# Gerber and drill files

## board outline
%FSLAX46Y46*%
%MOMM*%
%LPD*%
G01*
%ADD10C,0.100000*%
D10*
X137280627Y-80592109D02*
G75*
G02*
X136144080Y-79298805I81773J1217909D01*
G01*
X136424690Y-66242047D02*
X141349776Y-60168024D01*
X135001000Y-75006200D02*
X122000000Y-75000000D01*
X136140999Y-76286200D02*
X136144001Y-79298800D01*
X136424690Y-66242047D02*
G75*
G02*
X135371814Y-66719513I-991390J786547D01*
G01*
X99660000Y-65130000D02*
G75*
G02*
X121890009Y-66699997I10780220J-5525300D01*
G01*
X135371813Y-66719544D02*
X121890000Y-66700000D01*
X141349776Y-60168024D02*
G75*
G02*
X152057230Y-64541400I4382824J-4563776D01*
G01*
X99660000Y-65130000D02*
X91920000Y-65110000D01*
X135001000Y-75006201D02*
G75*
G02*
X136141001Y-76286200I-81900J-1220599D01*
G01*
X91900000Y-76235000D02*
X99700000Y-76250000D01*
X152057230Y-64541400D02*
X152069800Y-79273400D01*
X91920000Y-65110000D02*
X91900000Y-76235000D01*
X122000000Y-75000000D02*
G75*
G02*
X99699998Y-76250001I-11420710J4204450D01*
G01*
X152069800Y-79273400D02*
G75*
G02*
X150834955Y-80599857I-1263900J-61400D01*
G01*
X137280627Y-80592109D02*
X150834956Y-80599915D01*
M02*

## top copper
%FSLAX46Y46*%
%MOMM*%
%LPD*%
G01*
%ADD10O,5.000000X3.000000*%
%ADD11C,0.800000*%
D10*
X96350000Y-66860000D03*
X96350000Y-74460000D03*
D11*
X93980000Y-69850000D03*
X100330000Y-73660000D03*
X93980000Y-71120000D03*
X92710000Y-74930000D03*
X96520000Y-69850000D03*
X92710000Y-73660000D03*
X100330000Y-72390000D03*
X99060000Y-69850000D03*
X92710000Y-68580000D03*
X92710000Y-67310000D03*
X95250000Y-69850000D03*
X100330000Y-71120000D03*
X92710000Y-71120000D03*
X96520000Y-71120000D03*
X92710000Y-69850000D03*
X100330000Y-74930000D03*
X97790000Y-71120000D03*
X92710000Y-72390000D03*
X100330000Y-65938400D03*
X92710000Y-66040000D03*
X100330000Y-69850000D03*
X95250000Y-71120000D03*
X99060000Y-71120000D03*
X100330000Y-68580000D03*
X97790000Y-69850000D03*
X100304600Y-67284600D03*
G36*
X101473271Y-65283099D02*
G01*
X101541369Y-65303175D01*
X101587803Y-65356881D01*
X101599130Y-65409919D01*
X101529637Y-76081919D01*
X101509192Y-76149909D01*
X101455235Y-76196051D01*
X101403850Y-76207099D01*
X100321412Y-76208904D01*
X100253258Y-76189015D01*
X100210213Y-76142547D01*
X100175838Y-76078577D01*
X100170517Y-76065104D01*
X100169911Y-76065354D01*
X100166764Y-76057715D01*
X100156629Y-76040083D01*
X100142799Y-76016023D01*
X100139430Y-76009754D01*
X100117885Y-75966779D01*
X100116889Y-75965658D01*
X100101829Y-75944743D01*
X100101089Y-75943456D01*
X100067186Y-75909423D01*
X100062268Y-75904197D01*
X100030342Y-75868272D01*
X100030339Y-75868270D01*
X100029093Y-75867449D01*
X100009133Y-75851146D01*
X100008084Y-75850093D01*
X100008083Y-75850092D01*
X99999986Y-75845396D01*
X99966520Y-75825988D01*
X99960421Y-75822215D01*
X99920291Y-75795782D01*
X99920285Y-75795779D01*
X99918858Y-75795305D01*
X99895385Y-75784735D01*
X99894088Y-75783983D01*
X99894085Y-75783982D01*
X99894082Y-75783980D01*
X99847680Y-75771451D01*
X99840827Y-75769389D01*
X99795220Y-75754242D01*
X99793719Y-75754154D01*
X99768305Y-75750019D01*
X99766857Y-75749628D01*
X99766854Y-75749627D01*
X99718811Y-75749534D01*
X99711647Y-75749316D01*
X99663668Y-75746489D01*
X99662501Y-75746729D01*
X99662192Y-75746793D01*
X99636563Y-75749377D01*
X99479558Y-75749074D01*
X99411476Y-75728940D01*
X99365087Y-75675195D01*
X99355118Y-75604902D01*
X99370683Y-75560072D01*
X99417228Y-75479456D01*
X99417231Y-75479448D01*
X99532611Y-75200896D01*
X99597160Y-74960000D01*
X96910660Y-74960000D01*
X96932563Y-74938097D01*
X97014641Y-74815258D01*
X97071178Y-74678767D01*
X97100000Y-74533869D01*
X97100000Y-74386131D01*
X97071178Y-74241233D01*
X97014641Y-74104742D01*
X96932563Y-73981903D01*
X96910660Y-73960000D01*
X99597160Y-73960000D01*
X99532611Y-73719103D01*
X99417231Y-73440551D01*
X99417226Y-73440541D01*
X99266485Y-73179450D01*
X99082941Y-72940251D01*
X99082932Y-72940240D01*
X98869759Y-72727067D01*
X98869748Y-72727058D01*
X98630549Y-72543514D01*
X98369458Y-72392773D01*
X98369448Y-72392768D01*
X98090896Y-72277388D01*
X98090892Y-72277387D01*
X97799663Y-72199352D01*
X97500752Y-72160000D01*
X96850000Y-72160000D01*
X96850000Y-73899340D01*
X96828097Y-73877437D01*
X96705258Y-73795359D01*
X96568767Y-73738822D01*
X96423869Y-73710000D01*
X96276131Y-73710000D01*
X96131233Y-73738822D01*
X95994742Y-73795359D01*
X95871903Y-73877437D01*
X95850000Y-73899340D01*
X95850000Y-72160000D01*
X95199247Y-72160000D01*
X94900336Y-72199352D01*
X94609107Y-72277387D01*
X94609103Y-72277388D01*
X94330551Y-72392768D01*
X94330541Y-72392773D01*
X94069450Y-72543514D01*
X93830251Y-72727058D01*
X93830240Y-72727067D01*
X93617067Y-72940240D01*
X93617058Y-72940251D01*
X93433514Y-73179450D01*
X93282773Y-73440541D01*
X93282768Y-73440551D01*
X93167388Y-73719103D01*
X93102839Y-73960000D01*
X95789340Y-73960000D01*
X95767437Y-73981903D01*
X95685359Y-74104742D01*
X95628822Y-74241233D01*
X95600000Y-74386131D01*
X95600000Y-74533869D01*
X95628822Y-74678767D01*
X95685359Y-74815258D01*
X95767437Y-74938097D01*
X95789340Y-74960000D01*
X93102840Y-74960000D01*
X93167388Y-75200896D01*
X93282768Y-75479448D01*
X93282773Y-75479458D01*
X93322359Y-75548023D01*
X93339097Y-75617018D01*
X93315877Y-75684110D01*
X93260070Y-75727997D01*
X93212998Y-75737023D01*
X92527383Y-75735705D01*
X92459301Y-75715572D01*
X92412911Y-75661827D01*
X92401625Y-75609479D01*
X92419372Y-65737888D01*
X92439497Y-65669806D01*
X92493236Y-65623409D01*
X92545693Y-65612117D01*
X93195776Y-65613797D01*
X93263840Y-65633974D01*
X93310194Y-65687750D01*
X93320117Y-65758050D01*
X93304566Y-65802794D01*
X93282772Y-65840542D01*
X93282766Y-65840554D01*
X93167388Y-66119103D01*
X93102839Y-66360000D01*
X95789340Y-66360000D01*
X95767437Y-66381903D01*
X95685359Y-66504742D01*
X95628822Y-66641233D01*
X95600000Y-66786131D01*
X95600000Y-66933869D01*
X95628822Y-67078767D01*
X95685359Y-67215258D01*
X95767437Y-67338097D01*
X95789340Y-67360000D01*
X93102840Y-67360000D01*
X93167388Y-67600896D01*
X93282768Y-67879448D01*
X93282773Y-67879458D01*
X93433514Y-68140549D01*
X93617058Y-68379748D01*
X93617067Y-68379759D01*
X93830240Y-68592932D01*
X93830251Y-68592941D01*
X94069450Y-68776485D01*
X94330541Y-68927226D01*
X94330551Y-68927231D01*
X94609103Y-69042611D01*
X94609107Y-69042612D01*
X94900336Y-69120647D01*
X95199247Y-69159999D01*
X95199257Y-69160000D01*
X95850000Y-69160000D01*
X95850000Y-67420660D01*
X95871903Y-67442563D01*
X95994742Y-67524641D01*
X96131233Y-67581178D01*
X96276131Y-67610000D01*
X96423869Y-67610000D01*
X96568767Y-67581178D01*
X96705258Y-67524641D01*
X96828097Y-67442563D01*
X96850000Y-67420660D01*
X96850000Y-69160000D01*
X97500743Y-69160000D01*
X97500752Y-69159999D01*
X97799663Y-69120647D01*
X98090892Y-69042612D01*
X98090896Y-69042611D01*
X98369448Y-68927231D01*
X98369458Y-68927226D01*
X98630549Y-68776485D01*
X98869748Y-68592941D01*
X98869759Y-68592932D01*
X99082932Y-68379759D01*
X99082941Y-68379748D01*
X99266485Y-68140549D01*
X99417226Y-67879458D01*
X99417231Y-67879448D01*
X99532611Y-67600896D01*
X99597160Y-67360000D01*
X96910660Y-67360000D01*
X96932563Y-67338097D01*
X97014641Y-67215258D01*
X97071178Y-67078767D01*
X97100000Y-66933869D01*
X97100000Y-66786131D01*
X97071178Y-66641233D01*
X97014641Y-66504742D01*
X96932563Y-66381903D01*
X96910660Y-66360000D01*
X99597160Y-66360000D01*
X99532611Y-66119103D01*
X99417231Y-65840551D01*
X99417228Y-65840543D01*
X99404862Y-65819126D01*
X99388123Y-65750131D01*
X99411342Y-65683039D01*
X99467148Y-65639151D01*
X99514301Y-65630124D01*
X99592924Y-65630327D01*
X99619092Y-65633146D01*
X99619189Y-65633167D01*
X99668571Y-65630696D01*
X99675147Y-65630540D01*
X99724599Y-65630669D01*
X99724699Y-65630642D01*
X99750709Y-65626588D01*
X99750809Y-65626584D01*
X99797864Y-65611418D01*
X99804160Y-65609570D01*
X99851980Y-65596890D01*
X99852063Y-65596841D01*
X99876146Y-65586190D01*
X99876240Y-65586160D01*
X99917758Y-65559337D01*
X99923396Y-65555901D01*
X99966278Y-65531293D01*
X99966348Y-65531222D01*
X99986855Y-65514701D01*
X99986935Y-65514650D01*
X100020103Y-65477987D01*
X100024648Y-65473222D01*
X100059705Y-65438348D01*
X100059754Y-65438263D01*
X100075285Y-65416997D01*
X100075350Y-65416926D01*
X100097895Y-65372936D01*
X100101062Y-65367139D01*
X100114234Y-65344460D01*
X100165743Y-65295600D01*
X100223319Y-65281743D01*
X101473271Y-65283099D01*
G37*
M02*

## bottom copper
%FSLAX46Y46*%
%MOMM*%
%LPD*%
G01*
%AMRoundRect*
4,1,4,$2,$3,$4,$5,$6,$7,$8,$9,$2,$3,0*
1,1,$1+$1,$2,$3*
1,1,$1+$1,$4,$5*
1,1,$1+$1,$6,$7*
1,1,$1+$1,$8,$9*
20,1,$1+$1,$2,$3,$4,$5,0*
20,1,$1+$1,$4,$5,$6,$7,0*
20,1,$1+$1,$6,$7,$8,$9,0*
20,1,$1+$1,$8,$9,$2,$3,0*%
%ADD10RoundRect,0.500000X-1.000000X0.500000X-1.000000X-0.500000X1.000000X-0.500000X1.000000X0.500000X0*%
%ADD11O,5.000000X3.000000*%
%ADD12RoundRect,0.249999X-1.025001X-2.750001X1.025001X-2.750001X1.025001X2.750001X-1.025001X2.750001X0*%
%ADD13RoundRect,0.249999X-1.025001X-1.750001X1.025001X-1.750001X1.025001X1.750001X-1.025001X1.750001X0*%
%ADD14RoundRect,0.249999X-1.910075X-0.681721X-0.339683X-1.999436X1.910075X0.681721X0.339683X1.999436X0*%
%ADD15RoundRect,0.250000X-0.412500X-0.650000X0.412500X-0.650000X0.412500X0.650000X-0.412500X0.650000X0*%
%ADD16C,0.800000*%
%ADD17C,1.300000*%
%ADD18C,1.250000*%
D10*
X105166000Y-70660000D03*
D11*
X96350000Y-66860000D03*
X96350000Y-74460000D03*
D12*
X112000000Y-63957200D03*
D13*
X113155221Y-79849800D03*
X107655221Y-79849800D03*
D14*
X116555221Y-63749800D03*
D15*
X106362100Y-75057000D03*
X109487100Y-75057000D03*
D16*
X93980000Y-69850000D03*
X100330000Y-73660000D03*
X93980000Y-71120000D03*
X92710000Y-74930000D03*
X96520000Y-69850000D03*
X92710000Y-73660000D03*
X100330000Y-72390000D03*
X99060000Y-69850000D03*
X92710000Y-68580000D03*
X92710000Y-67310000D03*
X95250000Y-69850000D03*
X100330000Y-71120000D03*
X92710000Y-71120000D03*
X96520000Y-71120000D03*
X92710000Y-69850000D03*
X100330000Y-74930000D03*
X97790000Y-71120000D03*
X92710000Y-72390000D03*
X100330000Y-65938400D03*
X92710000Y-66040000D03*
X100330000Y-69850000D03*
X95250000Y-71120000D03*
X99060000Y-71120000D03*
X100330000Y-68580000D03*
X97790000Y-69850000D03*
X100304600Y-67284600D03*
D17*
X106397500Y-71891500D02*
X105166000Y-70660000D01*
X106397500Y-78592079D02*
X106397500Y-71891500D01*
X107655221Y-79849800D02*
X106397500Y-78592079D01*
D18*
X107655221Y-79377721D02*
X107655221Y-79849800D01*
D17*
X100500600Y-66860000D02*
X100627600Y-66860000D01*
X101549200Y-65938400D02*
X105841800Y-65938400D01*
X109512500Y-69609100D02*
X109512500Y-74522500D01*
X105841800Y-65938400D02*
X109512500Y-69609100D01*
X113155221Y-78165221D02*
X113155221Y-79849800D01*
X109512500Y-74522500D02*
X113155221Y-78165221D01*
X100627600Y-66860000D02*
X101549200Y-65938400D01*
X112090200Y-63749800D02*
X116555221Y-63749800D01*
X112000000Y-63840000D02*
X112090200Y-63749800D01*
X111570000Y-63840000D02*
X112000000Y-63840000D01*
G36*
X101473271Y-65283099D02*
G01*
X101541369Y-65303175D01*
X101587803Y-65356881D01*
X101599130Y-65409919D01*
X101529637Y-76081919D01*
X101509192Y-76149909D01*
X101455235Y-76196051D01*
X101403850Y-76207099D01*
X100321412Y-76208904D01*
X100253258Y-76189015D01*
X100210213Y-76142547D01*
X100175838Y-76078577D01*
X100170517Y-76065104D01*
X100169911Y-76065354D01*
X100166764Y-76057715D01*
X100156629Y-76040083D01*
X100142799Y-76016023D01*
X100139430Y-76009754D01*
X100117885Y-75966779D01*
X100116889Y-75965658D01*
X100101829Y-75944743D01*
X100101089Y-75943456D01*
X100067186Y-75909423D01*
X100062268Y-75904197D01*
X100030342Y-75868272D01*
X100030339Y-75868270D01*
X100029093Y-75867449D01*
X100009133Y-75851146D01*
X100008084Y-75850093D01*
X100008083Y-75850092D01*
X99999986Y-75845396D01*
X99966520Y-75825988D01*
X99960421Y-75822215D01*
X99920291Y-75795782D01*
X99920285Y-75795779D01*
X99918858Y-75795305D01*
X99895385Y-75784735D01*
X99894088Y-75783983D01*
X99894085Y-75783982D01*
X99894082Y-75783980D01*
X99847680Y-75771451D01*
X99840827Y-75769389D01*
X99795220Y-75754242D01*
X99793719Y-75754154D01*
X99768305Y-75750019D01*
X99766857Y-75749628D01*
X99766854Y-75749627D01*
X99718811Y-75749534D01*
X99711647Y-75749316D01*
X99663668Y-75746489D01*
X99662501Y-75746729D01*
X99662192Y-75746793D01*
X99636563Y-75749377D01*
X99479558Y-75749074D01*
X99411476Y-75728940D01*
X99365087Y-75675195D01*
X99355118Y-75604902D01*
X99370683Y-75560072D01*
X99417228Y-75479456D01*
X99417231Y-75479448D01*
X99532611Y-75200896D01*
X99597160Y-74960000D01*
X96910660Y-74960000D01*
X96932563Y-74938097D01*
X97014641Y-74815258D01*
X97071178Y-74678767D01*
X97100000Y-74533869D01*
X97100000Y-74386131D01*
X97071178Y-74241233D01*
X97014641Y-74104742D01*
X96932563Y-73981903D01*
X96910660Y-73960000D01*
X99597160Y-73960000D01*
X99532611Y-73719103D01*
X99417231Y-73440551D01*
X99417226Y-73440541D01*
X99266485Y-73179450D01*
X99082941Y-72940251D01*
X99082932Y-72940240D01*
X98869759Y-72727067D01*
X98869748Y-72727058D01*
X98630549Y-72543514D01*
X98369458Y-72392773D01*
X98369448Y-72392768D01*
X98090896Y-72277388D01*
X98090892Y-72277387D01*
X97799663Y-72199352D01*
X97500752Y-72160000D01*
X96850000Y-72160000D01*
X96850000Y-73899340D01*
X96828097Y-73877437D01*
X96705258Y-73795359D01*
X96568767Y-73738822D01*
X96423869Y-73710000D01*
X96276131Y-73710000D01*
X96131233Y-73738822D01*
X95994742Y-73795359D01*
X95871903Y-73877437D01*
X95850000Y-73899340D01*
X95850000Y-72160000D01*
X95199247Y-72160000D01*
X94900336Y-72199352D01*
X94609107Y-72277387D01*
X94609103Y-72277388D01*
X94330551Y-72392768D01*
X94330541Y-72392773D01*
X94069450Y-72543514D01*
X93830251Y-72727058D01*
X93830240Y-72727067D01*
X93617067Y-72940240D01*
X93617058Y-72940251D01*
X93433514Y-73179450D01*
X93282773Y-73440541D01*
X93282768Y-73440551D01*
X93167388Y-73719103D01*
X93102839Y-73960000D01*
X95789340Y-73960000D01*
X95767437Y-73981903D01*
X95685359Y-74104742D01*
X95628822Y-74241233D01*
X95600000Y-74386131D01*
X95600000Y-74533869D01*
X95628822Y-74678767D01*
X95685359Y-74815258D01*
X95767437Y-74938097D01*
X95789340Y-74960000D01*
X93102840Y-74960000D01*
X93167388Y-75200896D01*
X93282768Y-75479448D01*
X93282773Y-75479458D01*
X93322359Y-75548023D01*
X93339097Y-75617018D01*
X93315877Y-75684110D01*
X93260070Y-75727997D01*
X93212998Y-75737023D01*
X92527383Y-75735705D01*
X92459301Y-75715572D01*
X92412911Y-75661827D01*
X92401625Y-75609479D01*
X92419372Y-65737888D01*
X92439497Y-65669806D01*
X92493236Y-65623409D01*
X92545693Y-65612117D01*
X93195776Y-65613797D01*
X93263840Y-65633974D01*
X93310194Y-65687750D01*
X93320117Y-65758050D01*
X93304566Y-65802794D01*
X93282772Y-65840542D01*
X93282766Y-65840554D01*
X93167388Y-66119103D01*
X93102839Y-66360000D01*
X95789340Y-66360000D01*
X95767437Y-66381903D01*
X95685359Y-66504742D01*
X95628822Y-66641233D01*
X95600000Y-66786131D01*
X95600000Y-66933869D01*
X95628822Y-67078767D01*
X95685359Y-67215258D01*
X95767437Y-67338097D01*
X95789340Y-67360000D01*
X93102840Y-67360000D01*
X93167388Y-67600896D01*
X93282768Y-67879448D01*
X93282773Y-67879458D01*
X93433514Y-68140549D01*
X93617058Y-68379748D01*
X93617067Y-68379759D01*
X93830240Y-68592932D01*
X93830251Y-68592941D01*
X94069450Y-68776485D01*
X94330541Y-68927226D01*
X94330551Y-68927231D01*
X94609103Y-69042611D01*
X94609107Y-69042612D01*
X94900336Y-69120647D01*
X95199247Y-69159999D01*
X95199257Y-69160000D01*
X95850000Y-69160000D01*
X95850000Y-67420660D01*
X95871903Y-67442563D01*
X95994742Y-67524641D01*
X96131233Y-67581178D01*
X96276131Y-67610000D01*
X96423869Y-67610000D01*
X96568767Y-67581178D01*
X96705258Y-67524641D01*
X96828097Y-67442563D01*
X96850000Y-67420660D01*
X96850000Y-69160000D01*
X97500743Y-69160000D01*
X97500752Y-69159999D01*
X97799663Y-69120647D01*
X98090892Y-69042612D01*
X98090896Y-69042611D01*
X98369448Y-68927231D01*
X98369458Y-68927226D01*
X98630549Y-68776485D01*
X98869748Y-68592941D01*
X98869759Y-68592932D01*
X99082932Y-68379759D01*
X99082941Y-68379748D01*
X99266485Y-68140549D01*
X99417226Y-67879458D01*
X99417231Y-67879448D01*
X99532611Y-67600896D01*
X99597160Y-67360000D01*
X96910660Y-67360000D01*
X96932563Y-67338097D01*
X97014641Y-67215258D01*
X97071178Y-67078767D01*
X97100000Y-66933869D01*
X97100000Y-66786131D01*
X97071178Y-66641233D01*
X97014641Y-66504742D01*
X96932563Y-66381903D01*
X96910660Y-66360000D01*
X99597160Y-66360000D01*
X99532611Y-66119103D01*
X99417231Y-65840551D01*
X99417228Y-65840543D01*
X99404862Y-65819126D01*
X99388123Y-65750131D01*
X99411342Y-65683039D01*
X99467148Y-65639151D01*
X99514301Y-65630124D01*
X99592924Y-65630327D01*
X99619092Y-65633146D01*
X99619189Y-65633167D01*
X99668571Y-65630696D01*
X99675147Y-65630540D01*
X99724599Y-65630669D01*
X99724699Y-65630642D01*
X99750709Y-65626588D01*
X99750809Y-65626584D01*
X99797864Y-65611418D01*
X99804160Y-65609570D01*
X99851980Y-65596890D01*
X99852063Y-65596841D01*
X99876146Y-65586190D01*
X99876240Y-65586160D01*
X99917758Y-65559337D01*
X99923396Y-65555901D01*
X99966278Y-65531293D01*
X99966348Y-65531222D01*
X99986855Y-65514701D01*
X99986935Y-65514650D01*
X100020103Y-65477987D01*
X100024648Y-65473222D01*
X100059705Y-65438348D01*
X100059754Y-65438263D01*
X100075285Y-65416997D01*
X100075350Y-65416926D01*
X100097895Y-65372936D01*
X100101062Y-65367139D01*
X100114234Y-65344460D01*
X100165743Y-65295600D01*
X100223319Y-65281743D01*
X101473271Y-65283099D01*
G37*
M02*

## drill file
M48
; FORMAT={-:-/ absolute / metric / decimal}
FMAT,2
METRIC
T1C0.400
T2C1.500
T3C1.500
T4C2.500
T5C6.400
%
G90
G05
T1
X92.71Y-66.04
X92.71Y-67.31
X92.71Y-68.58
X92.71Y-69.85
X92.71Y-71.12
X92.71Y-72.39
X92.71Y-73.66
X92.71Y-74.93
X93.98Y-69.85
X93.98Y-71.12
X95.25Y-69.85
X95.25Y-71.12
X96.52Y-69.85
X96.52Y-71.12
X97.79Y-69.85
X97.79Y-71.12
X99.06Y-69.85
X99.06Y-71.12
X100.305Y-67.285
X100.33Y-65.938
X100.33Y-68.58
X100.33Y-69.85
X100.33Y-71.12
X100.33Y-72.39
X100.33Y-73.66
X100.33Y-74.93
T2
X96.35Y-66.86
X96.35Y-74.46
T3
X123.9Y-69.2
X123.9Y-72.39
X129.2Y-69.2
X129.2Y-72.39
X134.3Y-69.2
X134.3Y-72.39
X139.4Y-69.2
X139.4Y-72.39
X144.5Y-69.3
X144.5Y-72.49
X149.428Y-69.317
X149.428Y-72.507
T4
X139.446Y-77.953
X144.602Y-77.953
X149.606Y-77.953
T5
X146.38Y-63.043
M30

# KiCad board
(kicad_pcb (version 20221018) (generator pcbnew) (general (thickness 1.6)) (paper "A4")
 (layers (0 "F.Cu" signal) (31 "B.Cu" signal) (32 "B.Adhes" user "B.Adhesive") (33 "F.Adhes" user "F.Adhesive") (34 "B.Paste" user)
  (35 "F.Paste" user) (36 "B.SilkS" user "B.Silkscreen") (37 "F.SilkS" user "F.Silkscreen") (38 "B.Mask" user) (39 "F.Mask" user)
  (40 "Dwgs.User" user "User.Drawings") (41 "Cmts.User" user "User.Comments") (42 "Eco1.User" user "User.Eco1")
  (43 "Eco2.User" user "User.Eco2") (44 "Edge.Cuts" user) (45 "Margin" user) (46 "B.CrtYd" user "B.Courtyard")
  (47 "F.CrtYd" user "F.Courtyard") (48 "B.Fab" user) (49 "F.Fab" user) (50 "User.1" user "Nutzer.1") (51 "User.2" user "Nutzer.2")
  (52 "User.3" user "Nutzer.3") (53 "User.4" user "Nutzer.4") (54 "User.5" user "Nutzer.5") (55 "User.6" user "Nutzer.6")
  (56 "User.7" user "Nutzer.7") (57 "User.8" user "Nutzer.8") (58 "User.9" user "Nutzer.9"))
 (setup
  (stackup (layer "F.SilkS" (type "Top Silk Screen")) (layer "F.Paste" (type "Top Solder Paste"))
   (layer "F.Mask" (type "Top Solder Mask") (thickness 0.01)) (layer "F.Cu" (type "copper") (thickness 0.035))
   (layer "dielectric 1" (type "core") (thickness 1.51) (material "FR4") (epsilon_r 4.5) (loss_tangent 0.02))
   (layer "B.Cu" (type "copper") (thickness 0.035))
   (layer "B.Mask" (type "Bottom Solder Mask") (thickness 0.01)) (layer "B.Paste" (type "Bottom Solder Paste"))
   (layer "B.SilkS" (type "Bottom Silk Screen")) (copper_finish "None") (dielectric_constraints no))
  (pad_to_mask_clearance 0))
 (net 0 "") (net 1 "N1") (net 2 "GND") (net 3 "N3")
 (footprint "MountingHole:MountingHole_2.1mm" (layer "F.Cu") (at 149.4282 72.5066)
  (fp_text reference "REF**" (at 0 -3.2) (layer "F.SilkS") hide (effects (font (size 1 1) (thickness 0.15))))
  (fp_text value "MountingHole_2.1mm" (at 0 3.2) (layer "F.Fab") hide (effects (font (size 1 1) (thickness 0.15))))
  (pad "" np_thru_hole circle (at 0 0) (size 1.5 1.5) (drill 1.5) (layers "F&B.Cu" "*.Mask")))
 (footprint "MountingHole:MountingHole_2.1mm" (layer "F.Cu") (at 129.2 69.2)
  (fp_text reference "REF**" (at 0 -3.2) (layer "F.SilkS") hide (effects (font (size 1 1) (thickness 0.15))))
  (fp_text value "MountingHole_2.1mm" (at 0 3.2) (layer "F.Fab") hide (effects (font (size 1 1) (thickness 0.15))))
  (pad "" np_thru_hole circle (at 0 0) (size 1.5 1.5) (drill 1.5) (layers "F&B.Cu" "*.Mask")))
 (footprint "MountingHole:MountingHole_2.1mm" (layer "F.Cu") (at 144.5 72.49)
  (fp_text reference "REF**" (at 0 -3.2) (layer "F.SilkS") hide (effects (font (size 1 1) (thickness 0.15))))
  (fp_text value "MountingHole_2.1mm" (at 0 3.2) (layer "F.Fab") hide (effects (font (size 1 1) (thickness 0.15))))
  (pad "" np_thru_hole circle (at 0 0) (size 1.5 1.5) (drill 1.5) (layers "F&B.Cu" "*.Mask")))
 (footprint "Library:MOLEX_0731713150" (layer "F.Cu") (at 104.15 70.66 -90)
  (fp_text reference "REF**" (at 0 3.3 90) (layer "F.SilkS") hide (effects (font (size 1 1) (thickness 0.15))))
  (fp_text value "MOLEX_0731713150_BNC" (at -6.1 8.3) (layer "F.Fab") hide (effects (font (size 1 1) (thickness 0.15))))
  (pad "1" smd roundrect (at 0 -1.016 270) (size 2 3) (layers "B.Cu" "B.Paste" "B.Mask") (roundrect_rratio 0.25) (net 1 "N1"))
  (pad "2" thru_hole oval (at -3.8 7.8 270) (size 3 5) (drill 1.5) (layers "*.Cu" "*.Mask") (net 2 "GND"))
  (pad "2" thru_hole oval (at 3.8 7.8 270) (size 3 5) (drill 1.5) (layers "*.Cu" "*.Mask") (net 2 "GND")))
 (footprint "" (layer "F.Cu") (at 112 63.9572)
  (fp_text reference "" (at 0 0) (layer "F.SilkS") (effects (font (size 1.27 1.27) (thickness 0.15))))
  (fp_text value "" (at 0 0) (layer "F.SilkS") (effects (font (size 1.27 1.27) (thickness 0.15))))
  (pad "3" smd roundrect (at 0 0) (size 2.55 6) (layers "B.Cu" "B.Paste" "B.Mask") (roundrect_rratio 0.09803882353) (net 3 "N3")))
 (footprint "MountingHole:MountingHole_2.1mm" (layer "F.Cu") (at 134.3 69.2)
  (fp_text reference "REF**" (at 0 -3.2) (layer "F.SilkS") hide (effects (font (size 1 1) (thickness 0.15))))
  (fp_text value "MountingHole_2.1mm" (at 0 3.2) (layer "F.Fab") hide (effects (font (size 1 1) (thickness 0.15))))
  (pad "" np_thru_hole circle (at 0 0) (size 1.5 1.5) (drill 1.5) (layers "F&B.Cu" "*.Mask")))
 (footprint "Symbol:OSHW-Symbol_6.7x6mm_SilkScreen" (layer "F.Cu") (at 110.555221 70.7498 180)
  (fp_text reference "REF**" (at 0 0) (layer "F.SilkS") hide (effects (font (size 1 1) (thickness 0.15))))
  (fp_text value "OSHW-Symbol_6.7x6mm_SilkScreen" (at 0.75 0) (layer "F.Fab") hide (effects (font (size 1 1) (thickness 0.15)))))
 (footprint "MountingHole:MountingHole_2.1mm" (layer "F.Cu") (at 144.5 69.3)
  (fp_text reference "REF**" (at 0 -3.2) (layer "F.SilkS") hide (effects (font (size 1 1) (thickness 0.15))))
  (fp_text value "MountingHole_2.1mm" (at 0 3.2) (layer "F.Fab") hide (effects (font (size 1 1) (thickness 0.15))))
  (pad "" np_thru_hole circle (at 0 0) (size 1.5 1.5) (drill 1.5) (layers "F&B.Cu" "*.Mask")))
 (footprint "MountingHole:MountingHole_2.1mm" (layer "F.Cu") (at 123.9 72.39)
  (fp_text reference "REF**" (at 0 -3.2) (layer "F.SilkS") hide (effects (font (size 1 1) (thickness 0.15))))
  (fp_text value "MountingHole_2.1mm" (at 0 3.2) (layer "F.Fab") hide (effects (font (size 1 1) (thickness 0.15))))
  (pad "" np_thru_hole circle (at 0 0) (size 1.5 1.5) (drill 1.5) (layers "F&B.Cu" "*.Mask")))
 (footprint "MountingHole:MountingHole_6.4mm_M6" (layer "F.Cu") (at 146.3802 63.0428)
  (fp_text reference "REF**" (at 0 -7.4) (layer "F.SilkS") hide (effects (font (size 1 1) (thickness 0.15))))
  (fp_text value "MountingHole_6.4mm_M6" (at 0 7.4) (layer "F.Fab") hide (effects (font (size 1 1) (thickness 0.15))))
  (pad "" np_thru_hole circle (at 0 0) (size 6.4 6.4) (drill 6.4) (layers "*.Cu" "*.Mask")))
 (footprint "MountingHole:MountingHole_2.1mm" (layer "F.Cu") (at 129.2 72.39)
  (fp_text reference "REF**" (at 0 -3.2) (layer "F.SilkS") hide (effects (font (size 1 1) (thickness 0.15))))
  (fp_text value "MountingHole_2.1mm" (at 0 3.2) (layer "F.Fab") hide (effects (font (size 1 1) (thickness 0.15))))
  (pad "" np_thru_hole circle (at 0 0) (size 1.5 1.5) (drill 1.5) (layers "F&B.Cu" "*.Mask")))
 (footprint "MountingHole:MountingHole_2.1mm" (layer "F.Cu") (at 149.4282 69.3166)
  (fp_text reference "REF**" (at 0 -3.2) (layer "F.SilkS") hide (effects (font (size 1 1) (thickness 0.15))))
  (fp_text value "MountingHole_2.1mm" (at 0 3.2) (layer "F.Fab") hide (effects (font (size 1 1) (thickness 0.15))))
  (pad "" np_thru_hole circle (at 0 0) (size 1.5 1.5) (drill 1.5) (layers "F&B.Cu" "*.Mask")))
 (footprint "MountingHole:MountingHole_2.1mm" (layer "F.Cu") (at 123.9 69.2)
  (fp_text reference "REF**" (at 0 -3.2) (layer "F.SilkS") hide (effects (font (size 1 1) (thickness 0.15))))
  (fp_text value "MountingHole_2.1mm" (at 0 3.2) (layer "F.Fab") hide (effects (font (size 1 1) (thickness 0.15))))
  (pad "" np_thru_hole circle (at 0 0) (size 1.5 1.5) (drill 1.5) (layers "F&B.Cu" "*.Mask")))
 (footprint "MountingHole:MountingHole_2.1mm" (layer "F.Cu") (at 139.446 77.9526)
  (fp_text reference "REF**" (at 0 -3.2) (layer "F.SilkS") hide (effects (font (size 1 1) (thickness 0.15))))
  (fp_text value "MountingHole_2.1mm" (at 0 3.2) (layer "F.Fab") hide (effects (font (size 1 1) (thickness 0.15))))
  (pad "" np_thru_hole circle (at 0 0) (size 2.1 2.1) (drill 2.5) (layers "F&B.Cu" "*.Mask")))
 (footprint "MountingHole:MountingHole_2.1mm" (layer "F.Cu") (at 149.606 77.9526)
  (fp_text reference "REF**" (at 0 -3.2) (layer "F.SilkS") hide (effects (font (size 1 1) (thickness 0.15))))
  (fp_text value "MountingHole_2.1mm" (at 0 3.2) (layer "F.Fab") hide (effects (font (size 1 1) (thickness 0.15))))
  (pad "" np_thru_hole circle (at 0 0) (size 2.1 2.1) (drill 2.5) (layers "F&B.Cu" "*.Mask")))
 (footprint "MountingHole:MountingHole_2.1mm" (layer "F.Cu") (at 139.4 69.2)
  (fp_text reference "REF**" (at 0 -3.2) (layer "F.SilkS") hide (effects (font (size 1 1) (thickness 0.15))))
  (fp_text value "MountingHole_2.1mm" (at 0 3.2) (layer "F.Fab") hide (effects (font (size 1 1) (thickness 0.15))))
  (pad "" np_thru_hole circle (at 0 0) (size 1.5 1.5) (drill 1.5) (layers "F&B.Cu" "*.Mask")))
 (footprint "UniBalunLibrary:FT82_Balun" (layer "F.Cu") (at 110.555221 70.7498)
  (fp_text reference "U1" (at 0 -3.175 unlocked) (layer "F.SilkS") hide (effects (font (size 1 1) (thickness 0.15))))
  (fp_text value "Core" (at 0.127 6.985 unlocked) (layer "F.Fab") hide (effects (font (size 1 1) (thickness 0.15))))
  (pad "1" smd roundrect (at 2.6 9.1) (size 2.55 4) (layers "B.Cu" "B.Paste" "B.Mask") (roundrect_rratio 0.09803882353) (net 2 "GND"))
  (pad "2" smd roundrect (at -2.9 9.1) (size 2.55 4) (layers "B.Cu" "B.Paste" "B.Mask") (roundrect_rratio 0.09803882353) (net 1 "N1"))
  (pad "3" smd roundrect (at 6 -7 320) (size 2.55 4) (layers "B.Cu" "B.Paste" "B.Mask") (roundrect_rratio 0.09803882353) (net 3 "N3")))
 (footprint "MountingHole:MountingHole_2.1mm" (layer "F.Cu") (at 134.3 72.39)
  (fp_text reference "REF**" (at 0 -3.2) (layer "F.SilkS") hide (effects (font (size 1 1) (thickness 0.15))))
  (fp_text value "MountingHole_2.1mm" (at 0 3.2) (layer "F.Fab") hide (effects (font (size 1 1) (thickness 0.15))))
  (pad "" np_thru_hole circle (at 0 0) (size 1.5 1.5) (drill 1.5) (layers "F&B.Cu" "*.Mask")))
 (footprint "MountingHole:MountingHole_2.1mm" (layer "F.Cu") (at 139.4 72.39)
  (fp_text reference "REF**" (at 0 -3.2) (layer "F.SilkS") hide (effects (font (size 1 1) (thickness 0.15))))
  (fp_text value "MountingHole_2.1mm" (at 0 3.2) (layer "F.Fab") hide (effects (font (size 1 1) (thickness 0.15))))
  (pad "" np_thru_hole circle (at 0 0) (size 1.5 1.5) (drill 1.5) (layers "F&B.Cu" "*.Mask")))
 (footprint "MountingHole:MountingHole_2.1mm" (layer "F.Cu") (at 144.6022 77.9526)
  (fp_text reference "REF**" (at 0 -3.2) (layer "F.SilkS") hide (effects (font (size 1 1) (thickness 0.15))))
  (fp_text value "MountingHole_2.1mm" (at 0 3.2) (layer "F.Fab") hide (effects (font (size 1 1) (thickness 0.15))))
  (pad "" np_thru_hole circle (at 0 0) (size 2.1 2.1) (drill 2.5) (layers "F&B.Cu" "*.Mask")))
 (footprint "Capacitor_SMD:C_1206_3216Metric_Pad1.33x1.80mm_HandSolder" (layer "B.Cu") (at 107.9246 75.057)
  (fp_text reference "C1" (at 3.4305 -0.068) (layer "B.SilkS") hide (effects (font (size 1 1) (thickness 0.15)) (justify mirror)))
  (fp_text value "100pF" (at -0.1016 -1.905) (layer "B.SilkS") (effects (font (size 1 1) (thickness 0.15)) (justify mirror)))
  (pad "1" smd roundrect (at -1.5625 0) (size 1.325 1.8) (layers "B.Cu" "B.Paste" "B.Mask") (roundrect_rratio 0.1886792453) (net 1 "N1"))
  (pad "2" smd roundrect (at 1.5625 0) (size 1.325 1.8) (layers "B.Cu" "B.Paste" "B.Mask") (roundrect_rratio 0.1886792453) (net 2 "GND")))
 (gr_arc (start 137.280627 80.592109) (mid 136.445449 80.179989) (end 136.144001 79.2988) (stroke (width 0.1) (type solid))
  (layer "Edge.Cuts"))
 (gr_line (start 136.42469 66.242047) (end 141.349776 60.168024) (stroke (width 0.1) (type default)) (layer "Edge.Cuts"))
 (gr_line (start 135.001 75.0062) (end 122 75) (stroke (width 0.1) (type solid)) (layer "Edge.Cuts"))
 (gr_line (start 136.140999 76.2862) (end 136.144001 79.2988) (stroke (width 0.1) (type default)) (layer "Edge.Cuts"))
 (gr_arc (start 136.42469 66.242047) (mid 135.955963 66.608049) (end 135.371813 66.719544) (stroke (width 0.1) (type solid))
  (layer "Edge.Cuts"))
 (gr_arc (start 99.66 65.13) (mid 111.293623 58.571687) (end 121.89 66.7) (stroke (width 0.1) (type solid)) (layer "Edge.Cuts"))
 (gr_line (start 135.371813 66.719544) (end 121.89 66.7) (stroke (width 0.1) (type solid)) (layer "Edge.Cuts"))
 (gr_arc (start 141.349776 60.168024) (mid 148.125142 58.874075) (end 152.05723 64.5414) (stroke (width 0.1) (type default))
  (layer "Edge.Cuts"))
 (gr_line (start 99.66 65.13) (end 91.92 65.11) (stroke (width 0.1) (type solid)) (layer "Edge.Cuts"))
 (gr_arc (start 135.001 75.006201) (mid 135.832648 75.41317) (end 136.140999 76.2862) (stroke (width 0.1) (type solid)) (layer "Edge.Cuts"))
 (gr_line (start 91.9 76.235) (end 99.7 76.25) (stroke (width 0.1) (type solid)) (layer "Edge.Cuts"))
 (gr_line (start 152.05723 64.5414) (end 152.0698 79.2734) (stroke (width 0.1) (type solid)) (layer "Edge.Cuts"))
 (gr_line (start 91.92 65.11) (end 91.9 76.235) (stroke (width 0.1) (type solid)) (layer "Edge.Cuts"))
 (gr_arc (start 122 75) (mid 111.260399 82.946521) (end 99.7 76.25) (stroke (width 0.1) (type solid)) (layer "Edge.Cuts"))
 (gr_arc (start 152.0698 79.2734) (mid 151.732094 80.197043) (end 150.834956 80.599915) (stroke (width 0.1) (type solid))
  (layer "Edge.Cuts"))
 (gr_line (start 137.280627 80.592109) (end 150.834956 80.599915) (stroke (width 0.1) (type default)) (layer "Edge.Cuts"))
 (segment (start 106.3975 71.8915) (end 105.166 70.66) (width 1.3) (layer "B.Cu") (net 1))
 (segment (start 106.3975 78.592079) (end 106.3975 71.8915) (width 1.3) (layer "B.Cu") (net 1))
 (segment (start 107.655221 79.8498) (end 106.3975 78.592079) (width 1.3) (layer "B.Cu") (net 1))
 (segment (start 107.655221 79.377721) (end 107.655221 79.8498) (width 1.25) (layer "B.Cu") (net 1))
 (via (at 93.98 69.85) (size 0.8) (drill 0.4) (layers "F.Cu" "B.Cu") (free) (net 2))
 (via (at 100.33 73.66) (size 0.8) (drill 0.4) (layers "F.Cu" "B.Cu") (free) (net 2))
 (via (at 93.98 71.12) (size 0.8) (drill 0.4) (layers "F.Cu" "B.Cu") (free) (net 2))
 (via (at 92.71 74.93) (size 0.8) (drill 0.4) (layers "F.Cu" "B.Cu") (free) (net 2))
 (via (at 96.52 69.85) (size 0.8) (drill 0.4) (layers "F.Cu" "B.Cu") (free) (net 2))
 (via (at 92.71 73.66) (size 0.8) (drill 0.4) (layers "F.Cu" "B.Cu") (free) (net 2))
 (via (at 100.33 72.39) (size 0.8) (drill 0.4) (layers "F.Cu" "B.Cu") (free) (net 2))
 (via (at 99.06 69.85) (size 0.8) (drill 0.4) (layers "F.Cu" "B.Cu") (free) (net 2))
 (via (at 92.71 68.58) (size 0.8) (drill 0.4) (layers "F.Cu" "B.Cu") (free) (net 2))
 (via (at 92.71 67.31) (size 0.8) (drill 0.4) (layers "F.Cu" "B.Cu") (free) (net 2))
 (via (at 95.25 69.85) (size 0.8) (drill 0.4) (layers "F.Cu" "B.Cu") (free) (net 2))
 (via (at 100.33 71.12) (size 0.8) (drill 0.4) (layers "F.Cu" "B.Cu") (free) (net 2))
 (via (at 92.71 71.12) (size 0.8) (drill 0.4) (layers "F.Cu" "B.Cu") (free) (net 2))
 (via (at 96.52 71.12) (size 0.8) (drill 0.4) (layers "F.Cu" "B.Cu") (free) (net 2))
 (via (at 92.71 69.85) (size 0.8) (drill 0.4) (layers "F.Cu" "B.Cu") (free) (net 2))
 (via (at 100.33 74.93) (size 0.8) (drill 0.4) (layers "F.Cu" "B.Cu") (free) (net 2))
 (via (at 97.79 71.12) (size 0.8) (drill 0.4) (layers "F.Cu" "B.Cu") (free) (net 2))
 (via (at 92.71 72.39) (size 0.8) (drill 0.4) (layers "F.Cu" "B.Cu") (free) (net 2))
 (via (at 100.33 65.9384) (size 0.8) (drill 0.4) (layers "F.Cu" "B.Cu") (free) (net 2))
 (via (at 92.71 66.04) (size 0.8) (drill 0.4) (layers "F.Cu" "B.Cu") (free) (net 2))
 (via (at 100.33 69.85) (size 0.8) (drill 0.4) (layers "F.Cu" "B.Cu") (free) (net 2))
 (via (at 95.25 71.12) (size 0.8) (drill 0.4) (layers "F.Cu" "B.Cu") (free) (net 2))
 (via (at 99.06 71.12) (size 0.8) (drill 0.4) (layers "F.Cu" "B.Cu") (free) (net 2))
 (via (at 100.33 68.58) (size 0.8) (drill 0.4) (layers "F.Cu" "B.Cu") (free) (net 2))
 (via (at 97.79 69.85) (size 0.8) (drill 0.4) (layers "F.Cu" "B.Cu") (free) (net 2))
 (via (at 100.3046 67.2846) (size 0.8) (drill 0.4) (layers "F.Cu" "B.Cu") (free) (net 2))
 (segment (start 100.5006 66.86) (end 100.6276 66.86) (width 1.3) (layer "B.Cu") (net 2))
 (segment (start 101.5492 65.9384) (end 105.8418 65.9384) (width 1.3) (layer "B.Cu") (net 2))
 (segment (start 109.5125 69.6091) (end 109.5125 74.5225) (width 1.3) (layer "B.Cu") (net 2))
 (segment (start 105.8418 65.9384) (end 109.5125 69.6091) (width 1.3) (layer "B.Cu") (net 2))
 (segment (start 113.155221 78.165221) (end 113.155221 79.8498) (width 1.3) (layer "B.Cu") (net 2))
 (segment (start 109.5125 74.5225) (end 113.155221 78.165221) (width 1.3) (layer "B.Cu") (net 2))
 (segment (start 100.6276 66.86) (end 101.5492 65.9384) (width 1.3) (layer "B.Cu") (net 2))
 (segment (start 112.0902 63.7498) (end 116.555221 63.7498) (width 1.3) (layer "B.Cu") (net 3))
 (segment (start 112 63.84) (end 112.0902 63.7498) (width 1.3) (layer "B.Cu") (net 3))
 (segment (start 111.57 63.84) (end 112 63.84) (width 1.3) (layer "B.Cu") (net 3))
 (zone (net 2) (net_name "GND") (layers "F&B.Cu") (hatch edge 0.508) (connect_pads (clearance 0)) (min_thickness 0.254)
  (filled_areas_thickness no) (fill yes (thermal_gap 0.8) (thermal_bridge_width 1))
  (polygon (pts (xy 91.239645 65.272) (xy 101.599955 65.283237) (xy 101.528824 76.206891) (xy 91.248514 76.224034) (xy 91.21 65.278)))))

